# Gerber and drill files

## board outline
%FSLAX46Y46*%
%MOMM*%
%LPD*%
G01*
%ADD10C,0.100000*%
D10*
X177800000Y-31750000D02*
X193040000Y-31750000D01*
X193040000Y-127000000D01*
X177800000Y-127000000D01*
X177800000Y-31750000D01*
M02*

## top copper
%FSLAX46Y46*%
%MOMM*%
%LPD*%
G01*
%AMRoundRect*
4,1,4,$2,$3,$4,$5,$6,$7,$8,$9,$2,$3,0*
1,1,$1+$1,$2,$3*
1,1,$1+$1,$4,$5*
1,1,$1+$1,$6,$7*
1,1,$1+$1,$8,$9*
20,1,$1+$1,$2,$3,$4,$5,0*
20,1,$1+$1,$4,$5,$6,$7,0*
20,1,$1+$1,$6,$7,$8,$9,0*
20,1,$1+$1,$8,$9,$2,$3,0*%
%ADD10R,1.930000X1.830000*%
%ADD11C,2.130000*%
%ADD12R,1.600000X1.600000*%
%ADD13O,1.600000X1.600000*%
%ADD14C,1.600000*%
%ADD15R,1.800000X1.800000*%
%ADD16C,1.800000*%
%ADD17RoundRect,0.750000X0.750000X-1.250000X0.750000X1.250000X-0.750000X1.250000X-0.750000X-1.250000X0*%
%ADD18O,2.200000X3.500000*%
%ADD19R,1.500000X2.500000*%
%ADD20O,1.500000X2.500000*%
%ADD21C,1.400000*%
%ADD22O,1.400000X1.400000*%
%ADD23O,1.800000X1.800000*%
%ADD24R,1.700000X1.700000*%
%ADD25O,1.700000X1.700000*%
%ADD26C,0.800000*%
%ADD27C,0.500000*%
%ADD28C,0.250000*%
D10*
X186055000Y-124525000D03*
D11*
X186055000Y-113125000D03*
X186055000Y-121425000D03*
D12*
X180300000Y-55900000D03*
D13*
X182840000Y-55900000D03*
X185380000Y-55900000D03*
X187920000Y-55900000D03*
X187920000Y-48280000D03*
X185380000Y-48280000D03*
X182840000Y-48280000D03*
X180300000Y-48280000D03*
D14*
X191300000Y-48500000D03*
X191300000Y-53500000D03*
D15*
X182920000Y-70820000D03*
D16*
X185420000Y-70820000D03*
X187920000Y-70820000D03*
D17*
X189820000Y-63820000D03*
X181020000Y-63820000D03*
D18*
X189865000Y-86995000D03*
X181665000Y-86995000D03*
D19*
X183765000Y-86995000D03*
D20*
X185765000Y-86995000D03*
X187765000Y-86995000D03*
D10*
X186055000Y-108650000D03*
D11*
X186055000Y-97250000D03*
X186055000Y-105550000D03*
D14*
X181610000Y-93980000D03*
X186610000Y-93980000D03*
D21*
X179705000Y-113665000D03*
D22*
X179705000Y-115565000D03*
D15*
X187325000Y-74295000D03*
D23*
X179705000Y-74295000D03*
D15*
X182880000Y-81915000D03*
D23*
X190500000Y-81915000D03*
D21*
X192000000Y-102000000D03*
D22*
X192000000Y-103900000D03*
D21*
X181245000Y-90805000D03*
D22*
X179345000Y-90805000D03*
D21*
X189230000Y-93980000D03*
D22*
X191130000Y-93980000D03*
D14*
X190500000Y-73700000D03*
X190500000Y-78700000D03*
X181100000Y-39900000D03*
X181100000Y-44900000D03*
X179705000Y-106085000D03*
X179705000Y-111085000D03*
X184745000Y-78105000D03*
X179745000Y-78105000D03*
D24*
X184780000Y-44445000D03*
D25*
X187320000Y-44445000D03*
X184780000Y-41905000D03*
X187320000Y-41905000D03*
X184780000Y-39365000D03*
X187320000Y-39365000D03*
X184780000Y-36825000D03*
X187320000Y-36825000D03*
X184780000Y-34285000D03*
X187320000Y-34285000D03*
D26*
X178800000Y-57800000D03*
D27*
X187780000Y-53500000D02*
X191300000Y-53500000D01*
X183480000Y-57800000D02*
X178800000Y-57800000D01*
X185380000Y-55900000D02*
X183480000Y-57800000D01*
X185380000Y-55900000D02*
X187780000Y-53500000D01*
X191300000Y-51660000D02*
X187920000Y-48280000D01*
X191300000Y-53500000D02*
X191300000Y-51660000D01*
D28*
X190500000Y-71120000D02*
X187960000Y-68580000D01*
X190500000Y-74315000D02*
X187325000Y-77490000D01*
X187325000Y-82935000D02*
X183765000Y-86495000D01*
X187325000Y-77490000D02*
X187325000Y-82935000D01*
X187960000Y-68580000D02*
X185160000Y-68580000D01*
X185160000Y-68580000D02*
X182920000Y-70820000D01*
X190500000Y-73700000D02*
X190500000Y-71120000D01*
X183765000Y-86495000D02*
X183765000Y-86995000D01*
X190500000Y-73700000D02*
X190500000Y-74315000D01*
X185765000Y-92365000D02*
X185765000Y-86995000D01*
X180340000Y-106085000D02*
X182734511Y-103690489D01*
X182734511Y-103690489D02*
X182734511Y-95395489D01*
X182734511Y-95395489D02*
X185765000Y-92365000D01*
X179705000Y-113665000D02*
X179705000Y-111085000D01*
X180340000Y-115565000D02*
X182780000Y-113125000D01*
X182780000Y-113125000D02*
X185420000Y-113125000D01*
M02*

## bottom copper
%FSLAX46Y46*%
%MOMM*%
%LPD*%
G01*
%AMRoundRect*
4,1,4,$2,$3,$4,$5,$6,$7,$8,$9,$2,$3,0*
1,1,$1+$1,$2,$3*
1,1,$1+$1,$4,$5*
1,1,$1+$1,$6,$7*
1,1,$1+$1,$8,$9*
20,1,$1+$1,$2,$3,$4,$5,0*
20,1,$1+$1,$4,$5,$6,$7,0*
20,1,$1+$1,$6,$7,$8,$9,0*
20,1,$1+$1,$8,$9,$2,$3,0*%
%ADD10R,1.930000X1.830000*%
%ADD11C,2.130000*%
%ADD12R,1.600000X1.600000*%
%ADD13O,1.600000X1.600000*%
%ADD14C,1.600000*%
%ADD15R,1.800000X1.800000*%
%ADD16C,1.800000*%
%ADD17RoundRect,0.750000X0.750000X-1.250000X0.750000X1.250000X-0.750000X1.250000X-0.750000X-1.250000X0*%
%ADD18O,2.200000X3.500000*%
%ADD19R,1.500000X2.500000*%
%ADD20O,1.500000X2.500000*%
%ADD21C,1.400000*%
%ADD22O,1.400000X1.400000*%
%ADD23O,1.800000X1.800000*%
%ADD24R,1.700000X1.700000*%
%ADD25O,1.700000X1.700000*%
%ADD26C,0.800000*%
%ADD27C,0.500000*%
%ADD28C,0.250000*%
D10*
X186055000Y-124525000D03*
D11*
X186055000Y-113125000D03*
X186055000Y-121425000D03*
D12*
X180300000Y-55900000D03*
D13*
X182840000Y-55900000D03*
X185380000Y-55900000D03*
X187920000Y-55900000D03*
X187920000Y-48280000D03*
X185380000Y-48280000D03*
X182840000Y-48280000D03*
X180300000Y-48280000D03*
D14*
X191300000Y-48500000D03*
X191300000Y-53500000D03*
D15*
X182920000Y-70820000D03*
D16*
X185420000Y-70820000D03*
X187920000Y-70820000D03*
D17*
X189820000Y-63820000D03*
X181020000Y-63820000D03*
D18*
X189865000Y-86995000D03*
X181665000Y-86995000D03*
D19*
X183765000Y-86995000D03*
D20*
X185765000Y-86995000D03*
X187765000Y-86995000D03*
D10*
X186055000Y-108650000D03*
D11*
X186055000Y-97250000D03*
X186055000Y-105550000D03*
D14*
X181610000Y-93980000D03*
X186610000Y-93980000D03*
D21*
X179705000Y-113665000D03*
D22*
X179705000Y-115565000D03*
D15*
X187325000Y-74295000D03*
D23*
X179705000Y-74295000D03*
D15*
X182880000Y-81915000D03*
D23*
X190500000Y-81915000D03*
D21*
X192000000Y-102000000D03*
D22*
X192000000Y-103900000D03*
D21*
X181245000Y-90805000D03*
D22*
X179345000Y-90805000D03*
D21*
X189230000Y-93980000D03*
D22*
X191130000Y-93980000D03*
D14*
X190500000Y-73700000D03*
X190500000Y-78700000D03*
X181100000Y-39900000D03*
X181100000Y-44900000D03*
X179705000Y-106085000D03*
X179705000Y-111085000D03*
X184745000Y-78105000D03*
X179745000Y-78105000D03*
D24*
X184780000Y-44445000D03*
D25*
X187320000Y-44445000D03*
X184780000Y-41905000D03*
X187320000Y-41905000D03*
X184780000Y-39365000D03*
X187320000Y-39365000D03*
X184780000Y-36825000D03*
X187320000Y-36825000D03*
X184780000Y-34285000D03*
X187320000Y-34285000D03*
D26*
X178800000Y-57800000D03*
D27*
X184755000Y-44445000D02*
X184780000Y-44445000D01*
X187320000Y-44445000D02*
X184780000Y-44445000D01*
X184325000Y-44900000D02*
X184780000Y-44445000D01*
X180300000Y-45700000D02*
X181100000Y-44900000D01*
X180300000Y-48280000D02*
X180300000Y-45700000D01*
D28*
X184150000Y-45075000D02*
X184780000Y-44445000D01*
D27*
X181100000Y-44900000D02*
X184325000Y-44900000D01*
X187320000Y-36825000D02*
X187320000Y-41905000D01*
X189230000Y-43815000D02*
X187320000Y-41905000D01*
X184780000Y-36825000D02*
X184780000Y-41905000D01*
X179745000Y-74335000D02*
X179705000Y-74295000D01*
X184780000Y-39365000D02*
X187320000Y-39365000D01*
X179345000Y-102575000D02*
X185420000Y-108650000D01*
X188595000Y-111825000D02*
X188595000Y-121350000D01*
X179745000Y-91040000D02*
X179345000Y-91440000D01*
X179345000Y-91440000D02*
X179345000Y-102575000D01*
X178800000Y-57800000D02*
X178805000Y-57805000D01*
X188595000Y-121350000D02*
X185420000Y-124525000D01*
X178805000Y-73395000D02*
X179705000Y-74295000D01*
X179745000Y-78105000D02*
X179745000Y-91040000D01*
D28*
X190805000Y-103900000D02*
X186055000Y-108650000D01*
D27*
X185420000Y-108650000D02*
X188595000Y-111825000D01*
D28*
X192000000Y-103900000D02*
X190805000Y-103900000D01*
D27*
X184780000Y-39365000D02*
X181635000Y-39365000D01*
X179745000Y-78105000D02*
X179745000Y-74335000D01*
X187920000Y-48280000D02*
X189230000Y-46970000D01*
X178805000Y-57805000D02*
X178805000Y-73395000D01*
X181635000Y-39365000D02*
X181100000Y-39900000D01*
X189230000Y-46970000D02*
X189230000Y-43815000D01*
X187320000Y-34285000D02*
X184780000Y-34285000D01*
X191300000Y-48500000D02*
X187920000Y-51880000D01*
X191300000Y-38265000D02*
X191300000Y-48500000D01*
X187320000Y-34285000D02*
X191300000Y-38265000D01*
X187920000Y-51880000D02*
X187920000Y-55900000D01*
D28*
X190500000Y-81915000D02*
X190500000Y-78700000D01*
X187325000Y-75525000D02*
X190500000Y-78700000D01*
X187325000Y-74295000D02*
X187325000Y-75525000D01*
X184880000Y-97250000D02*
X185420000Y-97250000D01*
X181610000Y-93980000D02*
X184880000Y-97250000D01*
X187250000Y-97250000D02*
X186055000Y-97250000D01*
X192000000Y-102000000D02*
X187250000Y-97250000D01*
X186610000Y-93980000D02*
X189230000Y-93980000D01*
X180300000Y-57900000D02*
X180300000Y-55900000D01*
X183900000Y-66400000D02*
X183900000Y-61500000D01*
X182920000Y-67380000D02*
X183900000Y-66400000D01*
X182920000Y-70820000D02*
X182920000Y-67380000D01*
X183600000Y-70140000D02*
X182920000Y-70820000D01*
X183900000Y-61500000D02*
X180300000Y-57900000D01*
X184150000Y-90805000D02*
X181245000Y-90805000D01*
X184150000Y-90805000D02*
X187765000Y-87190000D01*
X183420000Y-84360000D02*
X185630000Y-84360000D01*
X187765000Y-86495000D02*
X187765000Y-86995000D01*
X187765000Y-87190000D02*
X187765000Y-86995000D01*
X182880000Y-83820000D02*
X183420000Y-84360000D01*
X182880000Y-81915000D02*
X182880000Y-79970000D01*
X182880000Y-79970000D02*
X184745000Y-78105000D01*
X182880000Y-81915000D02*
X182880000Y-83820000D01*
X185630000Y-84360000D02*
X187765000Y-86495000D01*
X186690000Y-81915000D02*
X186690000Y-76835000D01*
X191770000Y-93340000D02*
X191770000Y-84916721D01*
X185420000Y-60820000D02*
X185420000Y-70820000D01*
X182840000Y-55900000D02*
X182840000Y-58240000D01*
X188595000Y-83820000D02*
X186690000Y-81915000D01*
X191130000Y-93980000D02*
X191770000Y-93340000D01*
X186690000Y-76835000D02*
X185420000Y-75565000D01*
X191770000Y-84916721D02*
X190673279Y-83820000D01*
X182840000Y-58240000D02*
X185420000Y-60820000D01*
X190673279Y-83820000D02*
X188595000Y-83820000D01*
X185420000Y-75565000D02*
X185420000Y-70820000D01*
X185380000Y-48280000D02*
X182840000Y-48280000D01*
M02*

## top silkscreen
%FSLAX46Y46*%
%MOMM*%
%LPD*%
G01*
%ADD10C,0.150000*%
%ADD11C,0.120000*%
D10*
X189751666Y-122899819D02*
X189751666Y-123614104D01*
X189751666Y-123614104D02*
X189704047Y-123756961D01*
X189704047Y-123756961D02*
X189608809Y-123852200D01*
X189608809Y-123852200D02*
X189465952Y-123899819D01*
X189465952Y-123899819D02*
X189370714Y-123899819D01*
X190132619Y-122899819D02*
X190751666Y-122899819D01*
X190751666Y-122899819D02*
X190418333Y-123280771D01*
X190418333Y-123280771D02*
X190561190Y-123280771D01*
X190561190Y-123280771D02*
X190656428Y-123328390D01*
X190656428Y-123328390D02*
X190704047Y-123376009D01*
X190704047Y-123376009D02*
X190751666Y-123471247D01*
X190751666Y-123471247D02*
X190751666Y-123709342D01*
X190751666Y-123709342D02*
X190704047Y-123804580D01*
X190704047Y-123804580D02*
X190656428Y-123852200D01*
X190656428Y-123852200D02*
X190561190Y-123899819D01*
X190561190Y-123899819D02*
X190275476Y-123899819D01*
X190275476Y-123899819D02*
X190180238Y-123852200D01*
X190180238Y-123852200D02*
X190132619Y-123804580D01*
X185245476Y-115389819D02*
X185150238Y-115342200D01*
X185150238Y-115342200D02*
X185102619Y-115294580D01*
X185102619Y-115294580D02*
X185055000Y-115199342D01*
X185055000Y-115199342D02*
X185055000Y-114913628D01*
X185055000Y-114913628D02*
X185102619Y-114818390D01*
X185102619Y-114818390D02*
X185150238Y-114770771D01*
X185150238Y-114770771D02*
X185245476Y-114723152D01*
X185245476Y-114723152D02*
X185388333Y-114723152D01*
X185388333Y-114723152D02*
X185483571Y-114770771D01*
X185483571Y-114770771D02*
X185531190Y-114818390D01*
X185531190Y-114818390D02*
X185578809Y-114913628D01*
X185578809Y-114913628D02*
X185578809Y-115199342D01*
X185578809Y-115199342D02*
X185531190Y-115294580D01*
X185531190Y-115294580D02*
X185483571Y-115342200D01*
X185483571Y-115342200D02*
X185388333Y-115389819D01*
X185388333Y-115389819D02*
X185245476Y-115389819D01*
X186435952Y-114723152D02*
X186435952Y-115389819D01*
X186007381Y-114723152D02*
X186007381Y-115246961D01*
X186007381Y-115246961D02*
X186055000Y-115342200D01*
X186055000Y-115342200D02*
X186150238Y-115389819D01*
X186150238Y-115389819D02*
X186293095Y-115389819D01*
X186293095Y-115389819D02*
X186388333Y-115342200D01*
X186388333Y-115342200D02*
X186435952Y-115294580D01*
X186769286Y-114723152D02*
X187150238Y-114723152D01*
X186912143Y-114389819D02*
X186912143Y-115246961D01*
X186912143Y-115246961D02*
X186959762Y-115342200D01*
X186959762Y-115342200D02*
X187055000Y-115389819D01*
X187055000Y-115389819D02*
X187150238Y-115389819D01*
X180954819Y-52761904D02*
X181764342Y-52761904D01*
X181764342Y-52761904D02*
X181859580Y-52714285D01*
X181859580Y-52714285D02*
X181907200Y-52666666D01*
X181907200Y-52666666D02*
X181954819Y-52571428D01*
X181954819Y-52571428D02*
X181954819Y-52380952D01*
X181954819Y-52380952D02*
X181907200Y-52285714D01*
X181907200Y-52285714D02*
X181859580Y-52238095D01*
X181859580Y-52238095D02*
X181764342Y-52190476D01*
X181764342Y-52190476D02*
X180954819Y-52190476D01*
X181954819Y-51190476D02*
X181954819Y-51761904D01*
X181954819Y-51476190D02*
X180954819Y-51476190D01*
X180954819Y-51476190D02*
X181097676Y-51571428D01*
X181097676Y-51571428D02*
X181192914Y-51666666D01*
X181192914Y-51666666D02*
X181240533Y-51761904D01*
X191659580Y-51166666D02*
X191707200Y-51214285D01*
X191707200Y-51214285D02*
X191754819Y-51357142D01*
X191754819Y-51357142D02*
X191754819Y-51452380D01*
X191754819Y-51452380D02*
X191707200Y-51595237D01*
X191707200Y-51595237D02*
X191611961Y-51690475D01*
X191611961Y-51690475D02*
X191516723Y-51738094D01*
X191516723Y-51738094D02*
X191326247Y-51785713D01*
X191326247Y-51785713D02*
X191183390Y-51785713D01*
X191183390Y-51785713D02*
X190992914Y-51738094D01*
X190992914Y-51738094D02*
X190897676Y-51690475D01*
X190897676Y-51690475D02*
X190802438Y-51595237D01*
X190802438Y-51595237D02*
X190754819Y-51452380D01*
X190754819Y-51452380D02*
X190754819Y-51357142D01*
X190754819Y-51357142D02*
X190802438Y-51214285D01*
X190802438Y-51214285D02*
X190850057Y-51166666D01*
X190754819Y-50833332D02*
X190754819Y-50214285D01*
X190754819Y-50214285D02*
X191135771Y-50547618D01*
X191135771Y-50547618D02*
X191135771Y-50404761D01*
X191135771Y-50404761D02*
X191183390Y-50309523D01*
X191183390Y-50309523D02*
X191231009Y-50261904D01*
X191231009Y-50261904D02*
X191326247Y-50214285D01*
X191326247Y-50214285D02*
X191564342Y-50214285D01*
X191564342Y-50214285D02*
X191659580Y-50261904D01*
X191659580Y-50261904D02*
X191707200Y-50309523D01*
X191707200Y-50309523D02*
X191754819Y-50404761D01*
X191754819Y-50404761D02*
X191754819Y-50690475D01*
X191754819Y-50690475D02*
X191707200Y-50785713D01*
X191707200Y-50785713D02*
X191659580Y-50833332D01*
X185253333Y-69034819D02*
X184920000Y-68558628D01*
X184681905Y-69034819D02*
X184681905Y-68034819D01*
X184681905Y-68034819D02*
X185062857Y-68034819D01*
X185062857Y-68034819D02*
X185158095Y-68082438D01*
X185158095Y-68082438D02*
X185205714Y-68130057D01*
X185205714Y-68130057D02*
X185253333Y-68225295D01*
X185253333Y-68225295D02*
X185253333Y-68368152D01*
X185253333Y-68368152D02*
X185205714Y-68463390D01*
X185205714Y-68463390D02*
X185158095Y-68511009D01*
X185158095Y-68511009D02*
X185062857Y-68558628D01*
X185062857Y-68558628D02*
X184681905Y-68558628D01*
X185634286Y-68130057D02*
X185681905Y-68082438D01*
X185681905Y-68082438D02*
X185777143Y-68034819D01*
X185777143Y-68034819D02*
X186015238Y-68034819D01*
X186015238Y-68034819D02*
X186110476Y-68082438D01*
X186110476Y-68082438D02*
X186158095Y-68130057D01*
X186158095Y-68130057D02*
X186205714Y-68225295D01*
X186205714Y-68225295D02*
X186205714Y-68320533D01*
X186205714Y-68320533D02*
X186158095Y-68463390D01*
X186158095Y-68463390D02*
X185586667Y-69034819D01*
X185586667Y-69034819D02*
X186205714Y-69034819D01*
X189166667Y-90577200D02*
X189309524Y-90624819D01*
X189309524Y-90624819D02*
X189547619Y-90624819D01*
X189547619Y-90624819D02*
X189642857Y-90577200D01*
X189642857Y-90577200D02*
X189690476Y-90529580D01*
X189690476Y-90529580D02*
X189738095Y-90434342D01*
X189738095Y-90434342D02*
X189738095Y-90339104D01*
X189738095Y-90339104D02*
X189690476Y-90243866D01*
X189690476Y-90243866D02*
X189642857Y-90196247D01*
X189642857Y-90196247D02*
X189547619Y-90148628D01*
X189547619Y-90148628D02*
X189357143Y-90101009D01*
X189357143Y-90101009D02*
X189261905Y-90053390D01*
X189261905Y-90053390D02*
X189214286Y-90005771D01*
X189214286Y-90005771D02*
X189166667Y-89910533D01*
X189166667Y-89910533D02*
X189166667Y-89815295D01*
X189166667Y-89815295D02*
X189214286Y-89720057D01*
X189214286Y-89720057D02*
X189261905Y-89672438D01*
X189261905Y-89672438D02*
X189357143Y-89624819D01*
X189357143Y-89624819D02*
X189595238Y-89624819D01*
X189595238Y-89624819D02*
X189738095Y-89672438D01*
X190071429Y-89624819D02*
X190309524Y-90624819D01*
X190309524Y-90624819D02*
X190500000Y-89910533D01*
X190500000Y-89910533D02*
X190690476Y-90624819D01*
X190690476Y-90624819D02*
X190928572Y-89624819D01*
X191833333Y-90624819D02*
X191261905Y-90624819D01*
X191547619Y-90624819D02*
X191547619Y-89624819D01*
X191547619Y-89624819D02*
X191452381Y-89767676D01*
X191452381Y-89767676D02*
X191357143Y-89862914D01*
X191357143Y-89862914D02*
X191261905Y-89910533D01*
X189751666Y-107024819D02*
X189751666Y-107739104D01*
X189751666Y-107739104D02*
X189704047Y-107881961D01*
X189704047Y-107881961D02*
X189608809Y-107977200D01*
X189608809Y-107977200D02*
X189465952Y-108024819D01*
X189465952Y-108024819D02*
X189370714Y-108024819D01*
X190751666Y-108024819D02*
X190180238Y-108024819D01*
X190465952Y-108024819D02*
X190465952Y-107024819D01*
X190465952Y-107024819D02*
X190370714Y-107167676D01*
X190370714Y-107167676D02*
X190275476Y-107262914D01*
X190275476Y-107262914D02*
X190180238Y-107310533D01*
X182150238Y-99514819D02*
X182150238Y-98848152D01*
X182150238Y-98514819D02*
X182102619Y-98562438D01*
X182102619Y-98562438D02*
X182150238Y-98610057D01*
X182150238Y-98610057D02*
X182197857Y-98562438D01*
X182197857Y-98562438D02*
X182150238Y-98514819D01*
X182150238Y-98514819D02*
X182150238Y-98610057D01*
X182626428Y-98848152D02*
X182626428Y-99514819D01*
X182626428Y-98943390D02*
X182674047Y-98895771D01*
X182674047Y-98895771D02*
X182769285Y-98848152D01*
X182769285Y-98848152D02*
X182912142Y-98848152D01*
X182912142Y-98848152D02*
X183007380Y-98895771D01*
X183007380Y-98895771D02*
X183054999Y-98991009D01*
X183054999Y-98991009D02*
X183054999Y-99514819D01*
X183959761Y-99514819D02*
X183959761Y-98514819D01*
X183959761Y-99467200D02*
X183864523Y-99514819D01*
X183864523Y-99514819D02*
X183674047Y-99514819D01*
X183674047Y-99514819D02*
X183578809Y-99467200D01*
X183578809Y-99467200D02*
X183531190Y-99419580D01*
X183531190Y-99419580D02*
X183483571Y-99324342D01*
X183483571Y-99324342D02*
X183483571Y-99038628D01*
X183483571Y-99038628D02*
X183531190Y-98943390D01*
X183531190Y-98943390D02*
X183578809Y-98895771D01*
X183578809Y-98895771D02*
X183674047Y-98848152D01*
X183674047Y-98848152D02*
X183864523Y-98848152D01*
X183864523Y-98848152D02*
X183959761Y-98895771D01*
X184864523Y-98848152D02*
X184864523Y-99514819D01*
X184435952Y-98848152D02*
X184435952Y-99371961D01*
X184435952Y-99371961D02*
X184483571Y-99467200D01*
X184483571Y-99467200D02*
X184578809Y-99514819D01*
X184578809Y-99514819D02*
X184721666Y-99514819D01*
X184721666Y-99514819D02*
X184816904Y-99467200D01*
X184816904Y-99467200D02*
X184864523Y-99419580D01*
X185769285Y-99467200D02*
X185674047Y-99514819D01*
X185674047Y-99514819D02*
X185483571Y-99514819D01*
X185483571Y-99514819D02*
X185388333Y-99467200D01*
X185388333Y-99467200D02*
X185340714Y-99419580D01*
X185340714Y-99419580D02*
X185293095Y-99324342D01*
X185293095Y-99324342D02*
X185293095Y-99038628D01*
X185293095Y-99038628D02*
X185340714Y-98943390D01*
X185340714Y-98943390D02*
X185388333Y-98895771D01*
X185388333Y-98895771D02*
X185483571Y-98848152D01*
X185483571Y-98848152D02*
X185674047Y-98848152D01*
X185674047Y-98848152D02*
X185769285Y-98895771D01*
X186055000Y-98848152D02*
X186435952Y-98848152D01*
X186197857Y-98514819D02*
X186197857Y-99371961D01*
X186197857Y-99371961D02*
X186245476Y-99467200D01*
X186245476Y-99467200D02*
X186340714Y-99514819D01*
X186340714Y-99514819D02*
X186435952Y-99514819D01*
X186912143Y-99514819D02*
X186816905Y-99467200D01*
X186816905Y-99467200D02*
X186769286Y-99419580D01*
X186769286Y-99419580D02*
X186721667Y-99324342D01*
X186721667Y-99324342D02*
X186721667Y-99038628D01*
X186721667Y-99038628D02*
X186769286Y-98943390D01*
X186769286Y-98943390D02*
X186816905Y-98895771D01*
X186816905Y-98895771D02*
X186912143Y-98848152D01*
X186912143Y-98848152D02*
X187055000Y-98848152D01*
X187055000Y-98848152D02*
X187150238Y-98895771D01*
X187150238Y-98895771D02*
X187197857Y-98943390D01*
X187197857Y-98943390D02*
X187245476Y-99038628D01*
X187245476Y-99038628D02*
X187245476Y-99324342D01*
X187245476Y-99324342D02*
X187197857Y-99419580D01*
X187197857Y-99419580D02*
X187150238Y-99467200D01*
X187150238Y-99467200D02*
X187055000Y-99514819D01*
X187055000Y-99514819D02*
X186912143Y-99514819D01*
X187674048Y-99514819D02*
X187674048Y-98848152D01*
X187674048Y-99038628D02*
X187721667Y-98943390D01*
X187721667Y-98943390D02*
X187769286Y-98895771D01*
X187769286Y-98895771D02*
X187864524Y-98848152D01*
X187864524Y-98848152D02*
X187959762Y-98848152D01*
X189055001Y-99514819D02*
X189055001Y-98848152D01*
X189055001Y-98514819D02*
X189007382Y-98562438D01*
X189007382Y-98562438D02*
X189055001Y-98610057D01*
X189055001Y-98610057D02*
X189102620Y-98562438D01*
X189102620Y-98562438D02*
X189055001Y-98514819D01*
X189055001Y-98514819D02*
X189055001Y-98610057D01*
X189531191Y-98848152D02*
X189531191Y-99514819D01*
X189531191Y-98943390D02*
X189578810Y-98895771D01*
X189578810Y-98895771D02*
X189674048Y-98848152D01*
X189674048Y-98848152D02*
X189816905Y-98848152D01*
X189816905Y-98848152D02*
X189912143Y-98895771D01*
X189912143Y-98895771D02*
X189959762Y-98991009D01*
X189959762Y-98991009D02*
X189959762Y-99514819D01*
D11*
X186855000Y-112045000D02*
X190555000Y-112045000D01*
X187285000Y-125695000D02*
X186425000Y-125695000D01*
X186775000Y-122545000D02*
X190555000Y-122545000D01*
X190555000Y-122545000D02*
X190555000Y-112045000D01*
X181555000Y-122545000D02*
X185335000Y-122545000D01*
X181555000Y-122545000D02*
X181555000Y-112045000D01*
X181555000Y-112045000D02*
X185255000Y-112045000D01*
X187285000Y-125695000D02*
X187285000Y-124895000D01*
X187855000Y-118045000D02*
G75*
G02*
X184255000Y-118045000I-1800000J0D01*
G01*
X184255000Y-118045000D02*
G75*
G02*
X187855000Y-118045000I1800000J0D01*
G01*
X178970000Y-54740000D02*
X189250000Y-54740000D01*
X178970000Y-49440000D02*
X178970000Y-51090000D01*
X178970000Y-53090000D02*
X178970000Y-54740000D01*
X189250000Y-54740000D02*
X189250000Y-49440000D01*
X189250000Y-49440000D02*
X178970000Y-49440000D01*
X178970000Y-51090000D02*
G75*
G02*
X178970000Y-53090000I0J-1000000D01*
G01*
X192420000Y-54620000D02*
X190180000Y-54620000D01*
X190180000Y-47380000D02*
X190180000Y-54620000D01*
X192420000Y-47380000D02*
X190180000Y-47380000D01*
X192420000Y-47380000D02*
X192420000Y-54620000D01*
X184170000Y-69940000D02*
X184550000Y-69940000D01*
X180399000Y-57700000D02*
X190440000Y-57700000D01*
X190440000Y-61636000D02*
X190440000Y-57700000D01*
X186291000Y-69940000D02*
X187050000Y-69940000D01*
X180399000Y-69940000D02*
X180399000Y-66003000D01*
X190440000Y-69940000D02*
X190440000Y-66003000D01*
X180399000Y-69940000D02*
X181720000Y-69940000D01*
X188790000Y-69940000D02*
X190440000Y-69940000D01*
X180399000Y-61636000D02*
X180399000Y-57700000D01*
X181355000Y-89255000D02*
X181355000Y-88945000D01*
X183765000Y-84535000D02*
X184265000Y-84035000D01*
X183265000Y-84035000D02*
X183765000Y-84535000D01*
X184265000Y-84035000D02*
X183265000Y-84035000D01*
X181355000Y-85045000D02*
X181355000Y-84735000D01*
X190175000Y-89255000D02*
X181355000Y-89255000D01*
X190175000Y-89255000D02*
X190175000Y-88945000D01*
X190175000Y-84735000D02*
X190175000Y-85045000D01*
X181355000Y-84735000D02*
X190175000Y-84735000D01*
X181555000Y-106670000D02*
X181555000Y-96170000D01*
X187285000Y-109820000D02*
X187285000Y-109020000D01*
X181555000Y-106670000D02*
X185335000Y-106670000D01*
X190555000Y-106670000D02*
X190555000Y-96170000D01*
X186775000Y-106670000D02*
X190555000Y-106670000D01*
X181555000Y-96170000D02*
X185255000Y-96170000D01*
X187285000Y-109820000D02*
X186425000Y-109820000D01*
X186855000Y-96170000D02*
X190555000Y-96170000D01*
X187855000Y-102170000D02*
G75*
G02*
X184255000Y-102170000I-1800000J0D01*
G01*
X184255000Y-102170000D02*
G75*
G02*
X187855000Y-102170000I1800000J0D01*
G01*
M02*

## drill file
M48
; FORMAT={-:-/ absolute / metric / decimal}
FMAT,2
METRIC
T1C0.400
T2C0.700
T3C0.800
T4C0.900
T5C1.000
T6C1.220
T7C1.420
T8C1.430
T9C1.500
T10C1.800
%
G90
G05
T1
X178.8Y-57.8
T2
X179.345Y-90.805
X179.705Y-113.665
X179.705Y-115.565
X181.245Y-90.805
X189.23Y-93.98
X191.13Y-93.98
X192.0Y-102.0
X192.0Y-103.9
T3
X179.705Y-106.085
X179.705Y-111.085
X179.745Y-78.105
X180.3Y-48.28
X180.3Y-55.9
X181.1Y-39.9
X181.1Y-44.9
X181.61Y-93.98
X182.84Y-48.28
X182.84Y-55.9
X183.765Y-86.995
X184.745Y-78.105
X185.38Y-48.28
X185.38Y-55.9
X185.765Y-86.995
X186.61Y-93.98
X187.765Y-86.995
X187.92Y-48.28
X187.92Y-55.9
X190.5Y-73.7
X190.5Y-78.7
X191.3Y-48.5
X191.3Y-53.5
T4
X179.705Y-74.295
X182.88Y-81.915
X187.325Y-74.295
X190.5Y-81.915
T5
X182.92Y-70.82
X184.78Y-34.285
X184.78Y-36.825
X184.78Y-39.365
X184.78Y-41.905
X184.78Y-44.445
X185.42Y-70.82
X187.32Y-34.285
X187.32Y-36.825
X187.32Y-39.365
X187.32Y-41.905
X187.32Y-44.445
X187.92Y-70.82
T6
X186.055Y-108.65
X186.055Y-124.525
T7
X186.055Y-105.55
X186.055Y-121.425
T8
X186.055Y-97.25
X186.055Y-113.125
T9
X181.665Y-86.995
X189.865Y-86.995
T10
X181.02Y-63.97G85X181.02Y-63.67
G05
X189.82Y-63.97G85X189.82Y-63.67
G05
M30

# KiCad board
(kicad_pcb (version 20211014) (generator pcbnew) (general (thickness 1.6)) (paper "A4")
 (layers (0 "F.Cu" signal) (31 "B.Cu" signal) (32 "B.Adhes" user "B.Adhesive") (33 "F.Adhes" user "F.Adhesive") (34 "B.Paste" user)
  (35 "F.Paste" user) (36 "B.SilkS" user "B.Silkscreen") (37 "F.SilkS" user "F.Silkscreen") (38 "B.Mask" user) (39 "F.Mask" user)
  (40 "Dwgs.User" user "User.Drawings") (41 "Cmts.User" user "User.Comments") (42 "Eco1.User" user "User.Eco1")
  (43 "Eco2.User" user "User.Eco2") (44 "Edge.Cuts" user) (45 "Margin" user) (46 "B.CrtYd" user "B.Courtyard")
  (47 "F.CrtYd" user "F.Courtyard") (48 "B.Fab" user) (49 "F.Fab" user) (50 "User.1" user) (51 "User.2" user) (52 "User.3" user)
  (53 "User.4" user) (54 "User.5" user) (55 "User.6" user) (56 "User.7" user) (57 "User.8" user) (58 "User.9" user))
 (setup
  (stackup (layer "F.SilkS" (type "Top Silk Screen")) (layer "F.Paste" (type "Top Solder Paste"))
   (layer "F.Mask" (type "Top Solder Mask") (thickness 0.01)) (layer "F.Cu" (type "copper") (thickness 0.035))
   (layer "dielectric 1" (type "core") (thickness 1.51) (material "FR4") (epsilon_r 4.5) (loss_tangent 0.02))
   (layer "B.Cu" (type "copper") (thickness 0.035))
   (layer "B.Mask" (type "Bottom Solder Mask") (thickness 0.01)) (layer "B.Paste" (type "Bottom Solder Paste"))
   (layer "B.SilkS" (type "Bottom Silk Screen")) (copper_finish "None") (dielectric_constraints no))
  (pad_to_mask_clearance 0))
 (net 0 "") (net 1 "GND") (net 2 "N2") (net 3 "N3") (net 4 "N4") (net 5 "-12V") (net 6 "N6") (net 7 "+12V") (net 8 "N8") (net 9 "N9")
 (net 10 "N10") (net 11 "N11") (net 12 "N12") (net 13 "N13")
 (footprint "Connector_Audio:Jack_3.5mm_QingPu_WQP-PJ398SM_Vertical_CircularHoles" (layer "F.Cu") (at 186.055 124.525 180)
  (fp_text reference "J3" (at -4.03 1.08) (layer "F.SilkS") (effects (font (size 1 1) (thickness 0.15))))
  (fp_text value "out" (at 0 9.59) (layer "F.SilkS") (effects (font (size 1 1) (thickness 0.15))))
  (fp_line (start -0.8 12.48) (end -4.5 12.48) (layer "F.SilkS") (width 0.12))
  (fp_line (start -1.23 -1.17) (end -0.37 -1.17) (layer "F.SilkS") (width 0.12))
  (fp_line (start -0.72 1.98) (end -4.5 1.98) (layer "F.SilkS") (width 0.12))
  (fp_line (start -4.5 1.98) (end -4.5 12.48) (layer "F.SilkS") (width 0.12))
  (fp_line (start 4.5 1.98) (end 0.72 1.98) (layer "F.SilkS") (width 0.12))
  (fp_line (start 4.5 1.98) (end 4.5 12.48) (layer "F.SilkS") (width 0.12))
  (fp_line (start 4.5 12.48) (end 0.8 12.48) (layer "F.SilkS") (width 0.12))
  (fp_line (start -1.23 -1.17) (end -1.23 -0.37) (layer "F.SilkS") (width 0.12))
  (fp_circle (center 0 6.48) (end 1.8 6.48) (layer "F.SilkS") (width 0.12) (fill none))
  (pad "S" thru_hole rect (at 0 0) (size 1.93 1.83) (drill 1.22) (layers *.Cu *.Mask) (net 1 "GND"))
  (pad "T" thru_hole circle (at 0 11.4) (size 2.13 2.13) (drill 1.43) (layers *.Cu *.Mask) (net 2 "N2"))
  (pad "TN" thru_hole circle (at 0 3.1) (size 2.13 2.13) (drill 1.42) (layers *.Cu *.Mask))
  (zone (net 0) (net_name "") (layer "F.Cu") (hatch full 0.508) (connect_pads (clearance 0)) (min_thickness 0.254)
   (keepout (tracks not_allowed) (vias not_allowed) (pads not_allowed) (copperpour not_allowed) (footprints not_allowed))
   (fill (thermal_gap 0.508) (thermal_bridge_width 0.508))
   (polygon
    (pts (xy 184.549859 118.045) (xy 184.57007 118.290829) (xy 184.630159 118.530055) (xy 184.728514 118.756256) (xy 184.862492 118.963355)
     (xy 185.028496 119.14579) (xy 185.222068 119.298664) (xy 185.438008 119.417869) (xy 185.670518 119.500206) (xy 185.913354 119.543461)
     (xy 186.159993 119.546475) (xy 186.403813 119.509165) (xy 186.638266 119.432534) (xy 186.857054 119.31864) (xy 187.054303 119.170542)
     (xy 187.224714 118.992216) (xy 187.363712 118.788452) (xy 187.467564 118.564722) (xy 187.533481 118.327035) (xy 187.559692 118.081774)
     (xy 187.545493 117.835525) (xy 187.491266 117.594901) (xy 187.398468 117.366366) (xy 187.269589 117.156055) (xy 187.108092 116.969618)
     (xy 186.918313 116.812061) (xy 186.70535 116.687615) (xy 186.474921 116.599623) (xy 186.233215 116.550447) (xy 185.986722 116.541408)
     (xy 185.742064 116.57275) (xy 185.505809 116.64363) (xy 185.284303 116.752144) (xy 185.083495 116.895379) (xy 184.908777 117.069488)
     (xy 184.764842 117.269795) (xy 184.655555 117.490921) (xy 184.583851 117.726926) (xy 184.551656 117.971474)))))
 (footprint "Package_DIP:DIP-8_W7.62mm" (layer "F.Cu") (at 180.3 55.9 90)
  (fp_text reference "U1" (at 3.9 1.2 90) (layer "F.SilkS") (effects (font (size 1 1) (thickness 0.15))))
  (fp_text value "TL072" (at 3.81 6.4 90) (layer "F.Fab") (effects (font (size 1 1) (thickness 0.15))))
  (fp_line (start 1.16 -1.33) (end 1.16 8.95) (layer "F.SilkS") (width 0.12))
  (fp_line (start 6.46 -1.33) (end 4.81 -1.33) (layer "F.SilkS") (width 0.12))
  (fp_line (start 2.81 -1.33) (end 1.16 -1.33) (layer "F.SilkS") (width 0.12))
  (fp_line (start 1.16 8.95) (end 6.46 8.95) (layer "F.SilkS") (width 0.12))
  (fp_line (start 6.46 8.95) (end 6.46 -1.33) (layer "F.SilkS") (width 0.12))
  (fp_arc (start 4.81 -1.33) (mid 3.81 -0.33) (end 2.81 -1.33) (layer "F.SilkS") (width 0.12))
  (pad "1" thru_hole rect (at 0 0 90) (size 1.6 1.6) (drill 0.8) (layers *.Cu *.Mask) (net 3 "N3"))
  (pad "2" thru_hole oval (at 0 2.54 90) (size 1.6 1.6) (drill 0.8) (layers *.Cu *.Mask) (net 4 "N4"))
  (pad "3" thru_hole oval (at 0 5.08 90) (size 1.6 1.6) (drill 0.8) (layers *.Cu *.Mask) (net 1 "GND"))
  (pad "4" thru_hole oval (at 0 7.62 90) (size 1.6 1.6) (drill 0.8) (layers *.Cu *.Mask) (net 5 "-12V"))
  (pad "5" thru_hole oval (at 7.62 7.62 90) (size 1.6 1.6) (drill 0.8) (layers *.Cu *.Mask) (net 1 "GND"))
  (pad "6" thru_hole oval (at 7.62 5.08 90) (size 1.6 1.6) (drill 0.8) (layers *.Cu *.Mask) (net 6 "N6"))
  (pad "7" thru_hole oval (at 7.62 2.54 90) (size 1.6 1.6) (drill 0.8) (layers *.Cu *.Mask) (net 6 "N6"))
  (pad "8" thru_hole oval (at 7.62 0 90) (size 1.6 1.6) (drill 0.8) (layers *.Cu *.Mask) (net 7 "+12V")))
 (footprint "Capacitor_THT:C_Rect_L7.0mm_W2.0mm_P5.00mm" (layer "F.Cu") (at 191.3 48.5 -90)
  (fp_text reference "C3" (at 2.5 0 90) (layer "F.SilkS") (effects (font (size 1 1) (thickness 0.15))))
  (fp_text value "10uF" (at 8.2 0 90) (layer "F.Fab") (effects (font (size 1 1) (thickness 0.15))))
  (fp_line (start 6.12 -1.12) (end 6.12 1.12) (layer "F.SilkS") (width 0.12))
  (fp_line (start -1.12 1.12) (end 6.12 1.12) (layer "F.SilkS") (width 0.12))
  (fp_line (start -1.12 -1.12) (end -1.12 1.12) (layer "F.SilkS") (width 0.12))
  (fp_line (start -1.12 -1.12) (end 6.12 -1.12) (layer "F.SilkS") (width 0.12))
  (pad "1" thru_hole circle (at 0 0 270) (size 1.6 1.6) (drill 0.8) (layers *.Cu *.Mask) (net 5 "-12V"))
  (pad "2" thru_hole circle (at 5 0 270) (size 1.6 1.6) (drill 0.8) (layers *.Cu *.Mask) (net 1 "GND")))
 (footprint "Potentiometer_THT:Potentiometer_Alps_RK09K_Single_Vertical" (layer "F.Cu") (at 182.92 70.82 90)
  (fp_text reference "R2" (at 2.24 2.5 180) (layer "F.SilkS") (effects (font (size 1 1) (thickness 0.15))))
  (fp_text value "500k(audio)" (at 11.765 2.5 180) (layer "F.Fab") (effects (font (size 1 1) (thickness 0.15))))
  (fp_line (start 0.88 1.25) (end 0.88 1.63) (layer "F.SilkS") (width 0.12))
  (fp_line (start 13.12 -2.521) (end 13.12 7.52) (layer "F.SilkS") (width 0.12))
  (fp_line (start 9.184 7.52) (end 13.12 7.52) (layer "F.SilkS") (width 0.12))
  (fp_line (start 0.88 3.371) (end 0.88 4.13) (layer "F.SilkS") (width 0.12))
  (fp_line (start 0.88 -2.521) (end 4.817 -2.521) (layer "F.SilkS") (width 0.12))
  (fp_line (start 0.88 7.52) (end 4.817 7.52) (layer "F.SilkS") (width 0.12))
  (fp_line (start 0.88 -2.521) (end 0.88 -1.2) (layer "F.SilkS") (width 0.12))
  (fp_line (start 0.88 5.87) (end 0.88 7.52) (layer "F.SilkS") (width 0.12))
  (fp_line (start 9.184 -2.521) (end 13.12 -2.521) (layer "F.SilkS") (width 0.12))
  (pad "1" thru_hole rect (at 0 0 90) (size 1.8 1.8) (drill 1) (layers *.Cu *.Mask) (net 3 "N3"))
  (pad "2" thru_hole circle (at 0 2.5 90) (size 1.8 1.8) (drill 1) (layers *.Cu *.Mask) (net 4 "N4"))
  (pad "3" thru_hole circle (at 0 5 90) (size 1.8 1.8) (drill 1) (layers *.Cu *.Mask))
  (pad "MP" thru_hole roundrect (at 7 6.9 90) (size 4 3) (drill oval 2.1 1.8) (layers *.Cu *.Mask) (roundrect_rratio 0.25))
  (pad "MP" thru_hole roundrect (at 7 -1.9 90) (size 4 3) (drill oval 2.1 1.8) (layers *.Cu *.Mask) (roundrect_rratio 0.25)))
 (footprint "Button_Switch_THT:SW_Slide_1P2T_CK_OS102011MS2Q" (layer "F.Cu") (at 183.765 86.995)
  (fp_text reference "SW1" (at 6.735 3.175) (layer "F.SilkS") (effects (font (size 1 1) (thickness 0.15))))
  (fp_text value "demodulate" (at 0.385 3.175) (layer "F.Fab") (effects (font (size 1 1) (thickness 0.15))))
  (fp_line (start -2.41 2.26) (end -2.41 1.95) (layer "F.SilkS") (width 0.12))
  (fp_line (start 0 -2.46) (end 0.5 -2.96) (layer "F.SilkS") (width 0.12))
  (fp_line (start -0.5 -2.96) (end 0 -2.46) (layer "F.SilkS") (width 0.12))
  (fp_line (start 0.5 -2.96) (end -0.5 -2.96) (layer "F.SilkS") (width 0.12))
  (fp_line (start -2.41 -1.95) (end -2.41 -2.26) (layer "F.SilkS") (width 0.12))
  (fp_line (start 6.41 2.26) (end -2.41 2.26) (layer "F.SilkS") (width 0.12))
  (fp_line (start 6.41 2.26) (end 6.41 1.95) (layer "F.SilkS") (width 0.12))
  (fp_line (start 6.41 -2.26) (end 6.41 -1.95) (layer "F.SilkS") (width 0.12))
  (fp_line (start -2.41 -2.26) (end 6.41 -2.26) (layer "F.SilkS") (width 0.12))
  (pad "" thru_hole oval (at 6.1 0) (size 2.2 3.5) (drill 1.5) (layers *.Cu *.Mask))
  (pad "" thru_hole oval (at -2.1 0) (size 2.2 3.5) (drill 1.5) (layers *.Cu *.Mask))
  (pad "1" thru_hole rect (at 0 0) (size 1.5 2.5) (drill 0.8) (layers *.Cu *.Mask) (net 3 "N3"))
  (pad "2" thru_hole oval (at 2 0) (size 1.5 2.5) (drill 0.8) (layers *.Cu *.Mask) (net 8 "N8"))
  (pad "3" thru_hole oval (at 4 0) (size 1.5 2.5) (drill 0.8) (layers *.Cu *.Mask) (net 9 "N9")))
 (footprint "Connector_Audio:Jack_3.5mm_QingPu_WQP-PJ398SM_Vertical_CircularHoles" (layer "F.Cu") (at 186.055 108.65 180)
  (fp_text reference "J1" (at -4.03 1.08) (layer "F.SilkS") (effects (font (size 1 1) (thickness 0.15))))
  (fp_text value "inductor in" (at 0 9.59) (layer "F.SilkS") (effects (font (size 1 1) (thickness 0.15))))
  (fp_line (start 4.5 1.98) (end 4.5 12.48) (layer "F.SilkS") (width 0.12))
  (fp_line (start -1.23 -1.17) (end -1.23 -0.37) (layer "F.SilkS") (width 0.12))
  (fp_line (start 4.5 1.98) (end 0.72 1.98) (layer "F.SilkS") (width 0.12))
  (fp_line (start -4.5 1.98) (end -4.5 12.48) (layer "F.SilkS") (width 0.12))
  (fp_line (start -0.72 1.98) (end -4.5 1.98) (layer "F.SilkS") (width 0.12))
  (fp_line (start 4.5 12.48) (end 0.8 12.48) (layer "F.SilkS") (width 0.12))
  (fp_line (start -1.23 -1.17) (end -0.37 -1.17) (layer "F.SilkS") (width 0.12))
  (fp_line (start -0.8 12.48) (end -4.5 12.48) (layer "F.SilkS") (width 0.12))
  (fp_circle (center 0 6.48) (end 1.8 6.48) (layer "F.SilkS") (width 0.12) (fill none))
  (pad "S" thru_hole rect (at 0 0) (size 1.93 1.83) (drill 1.22) (layers *.Cu *.Mask) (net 1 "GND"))
  (pad "T" thru_hole circle (at 0 11.4) (size 2.13 2.13) (drill 1.43) (layers *.Cu *.Mask) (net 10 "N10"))
  (pad "TN" thru_hole circle (at 0 3.1) (size 2.13 2.13) (drill 1.42) (layers *.Cu *.Mask))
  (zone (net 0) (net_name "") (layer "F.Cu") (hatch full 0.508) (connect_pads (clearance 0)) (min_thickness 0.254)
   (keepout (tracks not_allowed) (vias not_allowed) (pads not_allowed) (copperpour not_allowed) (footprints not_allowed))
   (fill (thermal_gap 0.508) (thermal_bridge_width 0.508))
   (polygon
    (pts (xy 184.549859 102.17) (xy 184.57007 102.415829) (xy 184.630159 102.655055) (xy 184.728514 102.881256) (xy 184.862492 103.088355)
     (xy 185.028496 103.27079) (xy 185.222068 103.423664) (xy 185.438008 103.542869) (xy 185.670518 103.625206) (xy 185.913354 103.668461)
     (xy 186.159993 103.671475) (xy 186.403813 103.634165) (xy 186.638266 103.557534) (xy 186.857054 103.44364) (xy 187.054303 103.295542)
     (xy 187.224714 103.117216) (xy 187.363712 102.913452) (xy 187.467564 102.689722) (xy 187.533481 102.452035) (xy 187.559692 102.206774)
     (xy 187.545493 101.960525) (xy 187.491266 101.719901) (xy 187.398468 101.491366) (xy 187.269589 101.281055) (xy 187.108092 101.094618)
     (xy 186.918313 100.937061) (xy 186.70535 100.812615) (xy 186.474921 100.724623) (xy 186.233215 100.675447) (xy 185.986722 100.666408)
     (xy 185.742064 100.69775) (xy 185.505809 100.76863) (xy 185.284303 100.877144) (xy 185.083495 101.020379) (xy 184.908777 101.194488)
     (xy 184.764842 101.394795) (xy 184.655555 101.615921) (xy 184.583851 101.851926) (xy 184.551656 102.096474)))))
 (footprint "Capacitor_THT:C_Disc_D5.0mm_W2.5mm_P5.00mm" (layer "B.Cu") (at 181.61 93.98)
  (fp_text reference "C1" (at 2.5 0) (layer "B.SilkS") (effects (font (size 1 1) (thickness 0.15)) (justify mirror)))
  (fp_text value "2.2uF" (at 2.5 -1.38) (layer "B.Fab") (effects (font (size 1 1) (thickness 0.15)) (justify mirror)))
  (pad "1" thru_hole circle (at 0 0) (size 1.6 1.6) (drill 0.8) (layers *.Cu *.Mask) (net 10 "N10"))
  (pad "2" thru_hole circle (at 5 0) (size 1.6 1.6) (drill 0.8) (layers *.Cu *.Mask) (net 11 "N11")))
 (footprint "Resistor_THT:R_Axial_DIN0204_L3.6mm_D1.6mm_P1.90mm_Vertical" (layer "B.Cu") (at 179.705 113.665 -90)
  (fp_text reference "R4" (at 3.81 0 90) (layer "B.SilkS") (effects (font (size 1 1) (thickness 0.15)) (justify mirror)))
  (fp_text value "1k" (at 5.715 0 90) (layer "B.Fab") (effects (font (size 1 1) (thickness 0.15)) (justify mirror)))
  (pad "1" thru_hole circle (at 0 0 270) (size 1.4 1.4) (drill 0.7) (layers *.Cu *.Mask) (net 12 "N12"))
  (pad "2" thru_hole oval (at 1.9 0 270) (size 1.4 1.4) (drill 0.7) (layers *.Cu *.Mask) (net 2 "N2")))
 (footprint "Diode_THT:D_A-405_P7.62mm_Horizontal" (layer "B.Cu") (at 187.325 74.295 180)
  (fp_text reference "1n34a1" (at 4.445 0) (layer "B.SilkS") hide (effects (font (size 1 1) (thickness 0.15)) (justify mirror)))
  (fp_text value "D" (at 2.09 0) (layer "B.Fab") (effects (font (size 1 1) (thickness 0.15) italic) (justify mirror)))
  (pad "1" thru_hole rect (at 0 0 180) (size 1.8 1.8) (drill 0.9) (layers *.Cu *.Mask) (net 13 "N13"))
  (pad "2" thru_hole oval (at 7.62 0 180) (size 1.8 1.8) (drill 0.9) (layers *.Cu *.Mask) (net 1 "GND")))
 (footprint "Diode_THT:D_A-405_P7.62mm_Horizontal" (layer "B.Cu") (at 182.88 81.915)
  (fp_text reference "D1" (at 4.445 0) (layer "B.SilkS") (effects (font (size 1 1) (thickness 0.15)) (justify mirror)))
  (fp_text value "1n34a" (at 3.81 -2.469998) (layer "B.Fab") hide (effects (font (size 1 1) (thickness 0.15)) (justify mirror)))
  (pad "1" thru_hole rect (at 0 0) (size 1.8 1.8) (drill 0.9) (layers *.Cu *.Mask) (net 9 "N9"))
  (pad "2" thru_hole oval (at 7.62 0) (size 1.8 1.8) (drill 0.9) (layers *.Cu *.Mask) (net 13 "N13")))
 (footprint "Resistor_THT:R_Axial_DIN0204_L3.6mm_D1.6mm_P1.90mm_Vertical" (layer "B.Cu") (at 192 102 -90)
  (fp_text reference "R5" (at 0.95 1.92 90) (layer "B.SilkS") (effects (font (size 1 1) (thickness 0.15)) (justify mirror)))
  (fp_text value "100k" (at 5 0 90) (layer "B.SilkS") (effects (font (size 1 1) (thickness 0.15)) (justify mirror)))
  (pad "1" thru_hole circle (at 0 0 270) (size 1.4 1.4) (drill 0.7) (layers *.Cu *.Mask) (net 10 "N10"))
  (pad "2" thru_hole oval (at 1.9 0 270) (size 1.4 1.4) (drill 0.7) (layers *.Cu *.Mask) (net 1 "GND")))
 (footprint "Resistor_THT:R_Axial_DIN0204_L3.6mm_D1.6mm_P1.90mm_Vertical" (layer "B.Cu") (at 181.245 90.805 180)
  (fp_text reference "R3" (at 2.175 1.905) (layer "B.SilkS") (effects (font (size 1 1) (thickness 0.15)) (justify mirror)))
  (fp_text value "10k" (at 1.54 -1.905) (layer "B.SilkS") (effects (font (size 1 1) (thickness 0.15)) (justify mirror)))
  (pad "1" thru_hole circle (at 0 0 180) (size 1.4 1.4) (drill 0.7) (layers *.Cu *.Mask) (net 9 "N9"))
  (pad "2" thru_hole oval (at 1.9 0 180) (size 1.4 1.4) (drill 0.7) (layers *.Cu *.Mask) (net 1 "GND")))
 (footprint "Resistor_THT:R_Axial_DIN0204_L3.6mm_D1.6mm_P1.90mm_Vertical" (layer "B.Cu") (at 189.23 93.98)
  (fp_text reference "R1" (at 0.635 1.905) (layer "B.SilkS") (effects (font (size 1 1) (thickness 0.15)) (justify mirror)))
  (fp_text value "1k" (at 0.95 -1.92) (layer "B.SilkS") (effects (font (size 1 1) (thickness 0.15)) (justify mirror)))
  (pad "1" thru_hole circle (at 0 0) (size 1.4 1.4) (drill 0.7) (layers *.Cu *.Mask) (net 11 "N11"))
  (pad "2" thru_hole oval (at 1.9 0) (size 1.4 1.4) (drill 0.7) (layers *.Cu *.Mask) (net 4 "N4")))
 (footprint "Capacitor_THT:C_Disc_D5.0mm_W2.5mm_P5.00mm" (layer "B.Cu") (at 190.5 73.7 -90)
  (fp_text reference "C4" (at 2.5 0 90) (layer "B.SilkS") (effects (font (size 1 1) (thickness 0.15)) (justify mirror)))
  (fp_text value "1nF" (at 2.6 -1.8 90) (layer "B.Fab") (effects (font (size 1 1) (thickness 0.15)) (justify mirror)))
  (pad "1" thru_hole circle (at 0 0 270) (size 1.6 1.6) (drill 0.8) (layers *.Cu *.Mask) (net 3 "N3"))
  (pad "2" thru_hole circle (at 5 0 270) (size 1.6 1.6) (drill 0.8) (layers *.Cu *.Mask) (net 13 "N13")))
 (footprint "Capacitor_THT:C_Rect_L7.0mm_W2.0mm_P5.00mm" (layer "B.Cu") (at 181.1 39.9 -90)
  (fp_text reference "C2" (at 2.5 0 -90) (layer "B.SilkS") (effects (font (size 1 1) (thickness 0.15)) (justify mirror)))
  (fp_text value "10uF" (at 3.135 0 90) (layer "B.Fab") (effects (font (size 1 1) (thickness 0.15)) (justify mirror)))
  (pad "1" thru_hole circle (at 0 0 270) (size 1.6 1.6) (drill 0.8) (layers *.Cu *.Mask) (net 1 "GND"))
  (pad "2" thru_hole circle (at 5 0 270) (size 1.6 1.6) (drill 0.8) (layers *.Cu *.Mask) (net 7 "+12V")))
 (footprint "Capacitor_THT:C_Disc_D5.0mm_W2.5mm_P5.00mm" (layer "B.Cu") (at 179.705 106.085 -90)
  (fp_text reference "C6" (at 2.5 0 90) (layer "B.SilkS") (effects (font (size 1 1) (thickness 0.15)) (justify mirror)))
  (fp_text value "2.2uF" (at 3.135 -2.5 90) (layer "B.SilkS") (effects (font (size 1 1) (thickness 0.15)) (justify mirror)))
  (pad "1" thru_hole circle (at 0 0 270) (size 1.6 1.6) (drill 0.8) (layers *.Cu *.Mask) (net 8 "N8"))
  (pad "2" thru_hole circle (at 5 0 270) (size 1.6 1.6) (drill 0.8) (layers *.Cu *.Mask) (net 12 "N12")))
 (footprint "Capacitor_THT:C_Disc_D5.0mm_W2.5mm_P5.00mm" (layer "B.Cu") (at 184.745 78.105 180)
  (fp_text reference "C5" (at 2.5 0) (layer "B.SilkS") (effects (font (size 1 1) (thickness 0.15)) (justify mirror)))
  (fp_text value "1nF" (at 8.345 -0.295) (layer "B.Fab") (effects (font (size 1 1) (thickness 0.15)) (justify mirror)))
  (pad "1" thru_hole circle (at 0 0 180) (size 1.6 1.6) (drill 0.8) (layers *.Cu *.Mask) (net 9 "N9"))
  (pad "2" thru_hole circle (at 5 0 180) (size 1.6 1.6) (drill 0.8) (layers *.Cu *.Mask) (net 1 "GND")))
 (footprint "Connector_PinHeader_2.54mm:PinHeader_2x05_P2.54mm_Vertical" (layer "B.Cu") (at 184.78 44.445)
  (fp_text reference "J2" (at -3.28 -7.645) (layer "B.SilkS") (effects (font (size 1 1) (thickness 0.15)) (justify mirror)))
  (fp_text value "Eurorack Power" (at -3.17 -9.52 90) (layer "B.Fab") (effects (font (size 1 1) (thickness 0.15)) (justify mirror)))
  (pad "1" thru_hole rect (at 0 0) (size 1.7 1.7) (drill 1) (layers *.Cu *.Mask) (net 7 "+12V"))
  (pad "2" thru_hole oval (at 2.54 0) (size 1.7 1.7) (drill 1) (layers *.Cu *.Mask) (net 7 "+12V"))
  (pad "3" thru_hole oval (at 0 -2.54) (size 1.7 1.7) (drill 1) (layers *.Cu *.Mask) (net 1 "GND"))
  (pad "4" thru_hole oval (at 2.54 -2.54) (size 1.7 1.7) (drill 1) (layers *.Cu *.Mask) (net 1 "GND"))
  (pad "5" thru_hole oval (at 0 -5.08) (size 1.7 1.7) (drill 1) (layers *.Cu *.Mask) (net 1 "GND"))
  (pad "6" thru_hole oval (at 2.54 -5.08) (size 1.7 1.7) (drill 1) (layers *.Cu *.Mask) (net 1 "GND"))
  (pad "7" thru_hole oval (at 0 -7.62) (size 1.7 1.7) (drill 1) (layers *.Cu *.Mask) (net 1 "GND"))
  (pad "8" thru_hole oval (at 2.54 -7.62) (size 1.7 1.7) (drill 1) (layers *.Cu *.Mask) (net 1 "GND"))
  (pad "9" thru_hole oval (at 0 -10.16) (size 1.7 1.7) (drill 1) (layers *.Cu *.Mask) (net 5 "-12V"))
  (pad "10" thru_hole oval (at 2.54 -10.16) (size 1.7 1.7) (drill 1) (layers *.Cu *.Mask) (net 5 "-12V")))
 (gr_rect (start 177.8 127) (end 193.04 31.75) (layer "Edge.Cuts") (width 0.1) (fill none))
 (segment (start 184.755 44.445) (end 184.78 44.445) (width 0.5) (layer "B.Cu") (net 7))
 (segment (start 187.32 44.445) (end 184.78 44.445) (width 0.5) (layer "B.Cu") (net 7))
 (segment (start 184.325 44.9) (end 184.78 44.445) (width 0.5) (layer "B.Cu") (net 7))
 (segment (start 180.3 45.7) (end 181.1 44.9) (width 0.5) (layer "B.Cu") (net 7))
 (segment (start 180.3 48.28) (end 180.3 45.7) (width 0.5) (layer "B.Cu") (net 7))
 (segment (start 184.15 45.075) (end 184.78 44.445) (width 0.25) (layer "B.Cu") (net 7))
 (segment (start 181.1 44.9) (end 184.325 44.9) (width 0.5) (layer "B.Cu") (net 7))
 (segment (start 187.78 53.5) (end 191.3 53.5) (width 0.5) (layer "F.Cu") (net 1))
 (segment (start 183.48 57.8) (end 178.8 57.8) (width 0.5) (layer "F.Cu") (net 1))
 (segment (start 185.38 55.9) (end 183.48 57.8) (width 0.5) (layer "F.Cu") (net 1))
 (segment (start 185.38 55.9) (end 187.78 53.5) (width 0.5) (layer "F.Cu") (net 1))
 (segment (start 191.3 51.66) (end 187.92 48.28) (width 0.5) (layer "F.Cu") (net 1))
 (segment (start 191.3 53.5) (end 191.3 51.66) (width 0.5) (layer "F.Cu") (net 1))
 (via (at 178.8 57.8) (size 0.8) (drill 0.4) (layers "F.Cu" "B.Cu") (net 1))
 (segment (start 187.32 36.825) (end 187.32 41.905) (width 0.5) (layer "B.Cu") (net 1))
 (segment (start 189.23 43.815) (end 187.32 41.905) (width 0.5) (layer "B.Cu") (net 1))
 (segment (start 184.78 36.825) (end 184.78 41.905) (width 0.5) (layer "B.Cu") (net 1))
 (segment (start 179.745 74.335) (end 179.705 74.295) (width 0.5) (layer "B.Cu") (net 1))
 (segment (start 184.78 39.365) (end 187.32 39.365) (width 0.5) (layer "B.Cu") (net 1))
 (segment (start 179.345 102.575) (end 185.42 108.65) (width 0.5) (layer "B.Cu") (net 1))
 (segment (start 188.595 111.825) (end 188.595 121.35) (width 0.5) (layer "B.Cu") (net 1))
 (segment (start 179.745 91.04) (end 179.345 91.44) (width 0.5) (layer "B.Cu") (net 1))
 (segment (start 179.345 91.44) (end 179.345 102.575) (width 0.5) (layer "B.Cu") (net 1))
 (segment (start 178.8 57.8) (end 178.805 57.805) (width 0.5) (layer "B.Cu") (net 1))
 (segment (start 188.595 121.35) (end 185.42 124.525) (width 0.5) (layer "B.Cu") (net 1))
 (segment (start 178.805 73.395) (end 179.705 74.295) (width 0.5) (layer "B.Cu") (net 1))
 (segment (start 179.745 78.105) (end 179.745 91.04) (width 0.5) (layer "B.Cu") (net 1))
 (segment (start 190.805 103.9) (end 186.055 108.65) (width 0.25) (layer "B.Cu") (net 1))
 (segment (start 185.42 108.65) (end 188.595 111.825) (width 0.5) (layer "B.Cu") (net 1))
 (segment (start 192 103.9) (end 190.805 103.9) (width 0.25) (layer "B.Cu") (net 1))
 (segment (start 184.78 39.365) (end 181.635 39.365) (width 0.5) (layer "B.Cu") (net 1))
 (segment (start 179.745 78.105) (end 179.745 74.335) (width 0.5) (layer "B.Cu") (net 1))
 (segment (start 187.92 48.28) (end 189.23 46.97) (width 0.5) (layer "B.Cu") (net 1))
 (segment (start 178.805 57.805) (end 178.805 73.395) (width 0.5) (layer "B.Cu") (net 1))
 (segment (start 181.635 39.365) (end 181.1 39.9) (width 0.5) (layer "B.Cu") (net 1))
 (segment (start 189.23 46.97) (end 189.23 43.815) (width 0.5) (layer "B.Cu") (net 1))
 (segment (start 187.32 34.285) (end 184.78 34.285) (width 0.5) (layer "B.Cu") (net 5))
 (segment (start 191.3 48.5) (end 187.92 51.88) (width 0.5) (layer "B.Cu") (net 5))
 (segment (start 191.3 38.265) (end 191.3 48.5) (width 0.5) (layer "B.Cu") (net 5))
 (segment (start 187.32 34.285) (end 191.3 38.265) (width 0.5) (layer "B.Cu") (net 5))
 (segment (start 187.92 51.88) (end 187.92 55.9) (width 0.5) (layer "B.Cu") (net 5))
 (segment (start 190.5 81.915) (end 190.5 78.7) (width 0.25) (layer "B.Cu") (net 13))
 (segment (start 187.325 75.525) (end 190.5 78.7) (width 0.25) (layer "B.Cu") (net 13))
 (segment (start 187.325 74.295) (end 187.325 75.525) (width 0.25) (layer "B.Cu") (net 13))
 (segment (start 184.88 97.25) (end 185.42 97.25) (width 0.25) (layer "B.Cu") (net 10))
 (segment (start 181.61 93.98) (end 184.88 97.25) (width 0.25) (layer "B.Cu") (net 10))
 (segment (start 187.25 97.25) (end 186.055 97.25) (width 0.25) (layer "B.Cu") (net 10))
 (segment (start 192 102) (end 187.25 97.25) (width 0.25) (layer "B.Cu") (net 10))
 (segment (start 186.61 93.98) (end 189.23 93.98) (width 0.25) (layer "B.Cu") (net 11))
 (segment (start 190.5 71.12) (end 187.96 68.58) (width 0.25) (layer "F.Cu") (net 3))
 (segment (start 190.5 74.315) (end 187.325 77.49) (width 0.25) (layer "F.Cu") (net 3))
 (segment (start 187.325 82.935) (end 183.765 86.495) (width 0.25) (layer "F.Cu") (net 3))
 (segment (start 187.325 77.49) (end 187.325 82.935) (width 0.25) (layer "F.Cu") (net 3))
 (segment (start 187.96 68.58) (end 185.16 68.58) (width 0.25) (layer "F.Cu") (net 3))
 (segment (start 185.16 68.58) (end 182.92 70.82) (width 0.25) (layer "F.Cu") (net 3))
 (segment (start 190.5 73.7) (end 190.5 71.12) (width 0.25) (layer "F.Cu") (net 3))
 (segment (start 183.765 86.495) (end 183.765 86.995) (width 0.25) (layer "F.Cu") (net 3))
 (segment (start 190.5 73.7) (end 190.5 74.315) (width 0.25) (layer "F.Cu") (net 3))
 (segment (start 180.3 57.9) (end 180.3 55.9) (width 0.25) (layer "B.Cu") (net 3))
 (segment (start 183.9 66.4) (end 183.9 61.5) (width 0.25) (layer "B.Cu") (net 3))
 (segment (start 182.92 67.38) (end 183.9 66.4) (width 0.25) (layer "B.Cu") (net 3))
 (segment (start 182.92 70.82) (end 182.92 67.38) (width 0.25) (layer "B.Cu") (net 3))
 (segment (start 183.6 70.14) (end 182.92 70.82) (width 0.25) (layer "B.Cu") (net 3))
 (segment (start 183.9 61.5) (end 180.3 57.9) (width 0.25) (layer "B.Cu") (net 3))
 (segment (start 184.15 90.805) (end 181.245 90.805) (width 0.25) (layer "B.Cu") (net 9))
 (segment (start 184.15 90.805) (end 187.765 87.19) (width 0.25) (layer "B.Cu") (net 9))
 (segment (start 183.42 84.36) (end 185.63 84.36) (width 0.25) (layer "B.Cu") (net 9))
 (segment (start 187.765 86.495) (end 187.765 86.995) (width 0.25) (layer "B.Cu") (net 9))
 (segment (start 187.765 87.19) (end 187.765 86.995) (width 0.25) (layer "B.Cu") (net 9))
 (segment (start 182.88 83.82) (end 183.42 84.36) (width 0.25) (layer "B.Cu") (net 9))
 (segment (start 182.88 81.915) (end 182.88 79.97) (width 0.25) (layer "B.Cu") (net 9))
 (segment (start 182.88 79.97) (end 184.745 78.105) (width 0.25) (layer "B.Cu") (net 9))
 (segment (start 182.88 81.915) (end 182.88 83.82) (width 0.25) (layer "B.Cu") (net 9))
 (segment (start 185.63 84.36) (end 187.765 86.495) (width 0.25) (layer "B.Cu") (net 9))
 (segment (start 185.765 92.365) (end 185.765 86.995) (width 0.25) (layer "F.Cu") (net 8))
 (segment (start 180.34 106.085) (end 182.734511 103.690489) (width 0.25) (layer "F.Cu") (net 8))
 (segment (start 182.734511 103.690489) (end 182.734511 95.395489) (width 0.25) (layer "F.Cu") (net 8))
 (segment (start 182.734511 95.395489) (end 185.765 92.365) (width 0.25) (layer "F.Cu") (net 8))
 (segment (start 179.705 113.665) (end 179.705 111.085) (width 0.25) (layer "F.Cu") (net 12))
 (segment (start 180.34 115.565) (end 182.78 113.125) (width 0.25) (layer "F.Cu") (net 2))
 (segment (start 182.78 113.125) (end 185.42 113.125) (width 0.25) (layer "F.Cu") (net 2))
 (segment (start 186.69 81.915) (end 186.69 76.835) (width 0.25) (layer "B.Cu") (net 4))
 (segment (start 191.77 93.34) (end 191.77 84.916721) (width 0.25) (layer "B.Cu") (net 4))
 (segment (start 185.42 60.82) (end 185.42 70.82) (width 0.25) (layer "B.Cu") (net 4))
 (segment (start 182.84 55.9) (end 182.84 58.24) (width 0.25) (layer "B.Cu") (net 4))
 (segment (start 188.595 83.82) (end 186.69 81.915) (width 0.25) (layer "B.Cu") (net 4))
 (segment (start 191.13 93.98) (end 191.77 93.34) (width 0.25) (layer "B.Cu") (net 4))
 (segment (start 186.69 76.835) (end 185.42 75.565) (width 0.25) (layer "B.Cu") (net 4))
 (segment (start 191.77 84.916721) (end 190.673279 83.82) (width 0.25) (layer "B.Cu") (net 4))
 (segment (start 182.84 58.24) (end 185.42 60.82) (width 0.25) (layer "B.Cu") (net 4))
 (segment (start 190.673279 83.82) (end 188.595 83.82) (width 0.25) (layer "B.Cu") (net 4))
 (segment (start 185.42 75.565) (end 185.42 70.82) (width 0.25) (layer "B.Cu") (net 4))
 (segment (start 185.38 48.28) (end 182.84 48.28) (width 0.25) (layer "B.Cu") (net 6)))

